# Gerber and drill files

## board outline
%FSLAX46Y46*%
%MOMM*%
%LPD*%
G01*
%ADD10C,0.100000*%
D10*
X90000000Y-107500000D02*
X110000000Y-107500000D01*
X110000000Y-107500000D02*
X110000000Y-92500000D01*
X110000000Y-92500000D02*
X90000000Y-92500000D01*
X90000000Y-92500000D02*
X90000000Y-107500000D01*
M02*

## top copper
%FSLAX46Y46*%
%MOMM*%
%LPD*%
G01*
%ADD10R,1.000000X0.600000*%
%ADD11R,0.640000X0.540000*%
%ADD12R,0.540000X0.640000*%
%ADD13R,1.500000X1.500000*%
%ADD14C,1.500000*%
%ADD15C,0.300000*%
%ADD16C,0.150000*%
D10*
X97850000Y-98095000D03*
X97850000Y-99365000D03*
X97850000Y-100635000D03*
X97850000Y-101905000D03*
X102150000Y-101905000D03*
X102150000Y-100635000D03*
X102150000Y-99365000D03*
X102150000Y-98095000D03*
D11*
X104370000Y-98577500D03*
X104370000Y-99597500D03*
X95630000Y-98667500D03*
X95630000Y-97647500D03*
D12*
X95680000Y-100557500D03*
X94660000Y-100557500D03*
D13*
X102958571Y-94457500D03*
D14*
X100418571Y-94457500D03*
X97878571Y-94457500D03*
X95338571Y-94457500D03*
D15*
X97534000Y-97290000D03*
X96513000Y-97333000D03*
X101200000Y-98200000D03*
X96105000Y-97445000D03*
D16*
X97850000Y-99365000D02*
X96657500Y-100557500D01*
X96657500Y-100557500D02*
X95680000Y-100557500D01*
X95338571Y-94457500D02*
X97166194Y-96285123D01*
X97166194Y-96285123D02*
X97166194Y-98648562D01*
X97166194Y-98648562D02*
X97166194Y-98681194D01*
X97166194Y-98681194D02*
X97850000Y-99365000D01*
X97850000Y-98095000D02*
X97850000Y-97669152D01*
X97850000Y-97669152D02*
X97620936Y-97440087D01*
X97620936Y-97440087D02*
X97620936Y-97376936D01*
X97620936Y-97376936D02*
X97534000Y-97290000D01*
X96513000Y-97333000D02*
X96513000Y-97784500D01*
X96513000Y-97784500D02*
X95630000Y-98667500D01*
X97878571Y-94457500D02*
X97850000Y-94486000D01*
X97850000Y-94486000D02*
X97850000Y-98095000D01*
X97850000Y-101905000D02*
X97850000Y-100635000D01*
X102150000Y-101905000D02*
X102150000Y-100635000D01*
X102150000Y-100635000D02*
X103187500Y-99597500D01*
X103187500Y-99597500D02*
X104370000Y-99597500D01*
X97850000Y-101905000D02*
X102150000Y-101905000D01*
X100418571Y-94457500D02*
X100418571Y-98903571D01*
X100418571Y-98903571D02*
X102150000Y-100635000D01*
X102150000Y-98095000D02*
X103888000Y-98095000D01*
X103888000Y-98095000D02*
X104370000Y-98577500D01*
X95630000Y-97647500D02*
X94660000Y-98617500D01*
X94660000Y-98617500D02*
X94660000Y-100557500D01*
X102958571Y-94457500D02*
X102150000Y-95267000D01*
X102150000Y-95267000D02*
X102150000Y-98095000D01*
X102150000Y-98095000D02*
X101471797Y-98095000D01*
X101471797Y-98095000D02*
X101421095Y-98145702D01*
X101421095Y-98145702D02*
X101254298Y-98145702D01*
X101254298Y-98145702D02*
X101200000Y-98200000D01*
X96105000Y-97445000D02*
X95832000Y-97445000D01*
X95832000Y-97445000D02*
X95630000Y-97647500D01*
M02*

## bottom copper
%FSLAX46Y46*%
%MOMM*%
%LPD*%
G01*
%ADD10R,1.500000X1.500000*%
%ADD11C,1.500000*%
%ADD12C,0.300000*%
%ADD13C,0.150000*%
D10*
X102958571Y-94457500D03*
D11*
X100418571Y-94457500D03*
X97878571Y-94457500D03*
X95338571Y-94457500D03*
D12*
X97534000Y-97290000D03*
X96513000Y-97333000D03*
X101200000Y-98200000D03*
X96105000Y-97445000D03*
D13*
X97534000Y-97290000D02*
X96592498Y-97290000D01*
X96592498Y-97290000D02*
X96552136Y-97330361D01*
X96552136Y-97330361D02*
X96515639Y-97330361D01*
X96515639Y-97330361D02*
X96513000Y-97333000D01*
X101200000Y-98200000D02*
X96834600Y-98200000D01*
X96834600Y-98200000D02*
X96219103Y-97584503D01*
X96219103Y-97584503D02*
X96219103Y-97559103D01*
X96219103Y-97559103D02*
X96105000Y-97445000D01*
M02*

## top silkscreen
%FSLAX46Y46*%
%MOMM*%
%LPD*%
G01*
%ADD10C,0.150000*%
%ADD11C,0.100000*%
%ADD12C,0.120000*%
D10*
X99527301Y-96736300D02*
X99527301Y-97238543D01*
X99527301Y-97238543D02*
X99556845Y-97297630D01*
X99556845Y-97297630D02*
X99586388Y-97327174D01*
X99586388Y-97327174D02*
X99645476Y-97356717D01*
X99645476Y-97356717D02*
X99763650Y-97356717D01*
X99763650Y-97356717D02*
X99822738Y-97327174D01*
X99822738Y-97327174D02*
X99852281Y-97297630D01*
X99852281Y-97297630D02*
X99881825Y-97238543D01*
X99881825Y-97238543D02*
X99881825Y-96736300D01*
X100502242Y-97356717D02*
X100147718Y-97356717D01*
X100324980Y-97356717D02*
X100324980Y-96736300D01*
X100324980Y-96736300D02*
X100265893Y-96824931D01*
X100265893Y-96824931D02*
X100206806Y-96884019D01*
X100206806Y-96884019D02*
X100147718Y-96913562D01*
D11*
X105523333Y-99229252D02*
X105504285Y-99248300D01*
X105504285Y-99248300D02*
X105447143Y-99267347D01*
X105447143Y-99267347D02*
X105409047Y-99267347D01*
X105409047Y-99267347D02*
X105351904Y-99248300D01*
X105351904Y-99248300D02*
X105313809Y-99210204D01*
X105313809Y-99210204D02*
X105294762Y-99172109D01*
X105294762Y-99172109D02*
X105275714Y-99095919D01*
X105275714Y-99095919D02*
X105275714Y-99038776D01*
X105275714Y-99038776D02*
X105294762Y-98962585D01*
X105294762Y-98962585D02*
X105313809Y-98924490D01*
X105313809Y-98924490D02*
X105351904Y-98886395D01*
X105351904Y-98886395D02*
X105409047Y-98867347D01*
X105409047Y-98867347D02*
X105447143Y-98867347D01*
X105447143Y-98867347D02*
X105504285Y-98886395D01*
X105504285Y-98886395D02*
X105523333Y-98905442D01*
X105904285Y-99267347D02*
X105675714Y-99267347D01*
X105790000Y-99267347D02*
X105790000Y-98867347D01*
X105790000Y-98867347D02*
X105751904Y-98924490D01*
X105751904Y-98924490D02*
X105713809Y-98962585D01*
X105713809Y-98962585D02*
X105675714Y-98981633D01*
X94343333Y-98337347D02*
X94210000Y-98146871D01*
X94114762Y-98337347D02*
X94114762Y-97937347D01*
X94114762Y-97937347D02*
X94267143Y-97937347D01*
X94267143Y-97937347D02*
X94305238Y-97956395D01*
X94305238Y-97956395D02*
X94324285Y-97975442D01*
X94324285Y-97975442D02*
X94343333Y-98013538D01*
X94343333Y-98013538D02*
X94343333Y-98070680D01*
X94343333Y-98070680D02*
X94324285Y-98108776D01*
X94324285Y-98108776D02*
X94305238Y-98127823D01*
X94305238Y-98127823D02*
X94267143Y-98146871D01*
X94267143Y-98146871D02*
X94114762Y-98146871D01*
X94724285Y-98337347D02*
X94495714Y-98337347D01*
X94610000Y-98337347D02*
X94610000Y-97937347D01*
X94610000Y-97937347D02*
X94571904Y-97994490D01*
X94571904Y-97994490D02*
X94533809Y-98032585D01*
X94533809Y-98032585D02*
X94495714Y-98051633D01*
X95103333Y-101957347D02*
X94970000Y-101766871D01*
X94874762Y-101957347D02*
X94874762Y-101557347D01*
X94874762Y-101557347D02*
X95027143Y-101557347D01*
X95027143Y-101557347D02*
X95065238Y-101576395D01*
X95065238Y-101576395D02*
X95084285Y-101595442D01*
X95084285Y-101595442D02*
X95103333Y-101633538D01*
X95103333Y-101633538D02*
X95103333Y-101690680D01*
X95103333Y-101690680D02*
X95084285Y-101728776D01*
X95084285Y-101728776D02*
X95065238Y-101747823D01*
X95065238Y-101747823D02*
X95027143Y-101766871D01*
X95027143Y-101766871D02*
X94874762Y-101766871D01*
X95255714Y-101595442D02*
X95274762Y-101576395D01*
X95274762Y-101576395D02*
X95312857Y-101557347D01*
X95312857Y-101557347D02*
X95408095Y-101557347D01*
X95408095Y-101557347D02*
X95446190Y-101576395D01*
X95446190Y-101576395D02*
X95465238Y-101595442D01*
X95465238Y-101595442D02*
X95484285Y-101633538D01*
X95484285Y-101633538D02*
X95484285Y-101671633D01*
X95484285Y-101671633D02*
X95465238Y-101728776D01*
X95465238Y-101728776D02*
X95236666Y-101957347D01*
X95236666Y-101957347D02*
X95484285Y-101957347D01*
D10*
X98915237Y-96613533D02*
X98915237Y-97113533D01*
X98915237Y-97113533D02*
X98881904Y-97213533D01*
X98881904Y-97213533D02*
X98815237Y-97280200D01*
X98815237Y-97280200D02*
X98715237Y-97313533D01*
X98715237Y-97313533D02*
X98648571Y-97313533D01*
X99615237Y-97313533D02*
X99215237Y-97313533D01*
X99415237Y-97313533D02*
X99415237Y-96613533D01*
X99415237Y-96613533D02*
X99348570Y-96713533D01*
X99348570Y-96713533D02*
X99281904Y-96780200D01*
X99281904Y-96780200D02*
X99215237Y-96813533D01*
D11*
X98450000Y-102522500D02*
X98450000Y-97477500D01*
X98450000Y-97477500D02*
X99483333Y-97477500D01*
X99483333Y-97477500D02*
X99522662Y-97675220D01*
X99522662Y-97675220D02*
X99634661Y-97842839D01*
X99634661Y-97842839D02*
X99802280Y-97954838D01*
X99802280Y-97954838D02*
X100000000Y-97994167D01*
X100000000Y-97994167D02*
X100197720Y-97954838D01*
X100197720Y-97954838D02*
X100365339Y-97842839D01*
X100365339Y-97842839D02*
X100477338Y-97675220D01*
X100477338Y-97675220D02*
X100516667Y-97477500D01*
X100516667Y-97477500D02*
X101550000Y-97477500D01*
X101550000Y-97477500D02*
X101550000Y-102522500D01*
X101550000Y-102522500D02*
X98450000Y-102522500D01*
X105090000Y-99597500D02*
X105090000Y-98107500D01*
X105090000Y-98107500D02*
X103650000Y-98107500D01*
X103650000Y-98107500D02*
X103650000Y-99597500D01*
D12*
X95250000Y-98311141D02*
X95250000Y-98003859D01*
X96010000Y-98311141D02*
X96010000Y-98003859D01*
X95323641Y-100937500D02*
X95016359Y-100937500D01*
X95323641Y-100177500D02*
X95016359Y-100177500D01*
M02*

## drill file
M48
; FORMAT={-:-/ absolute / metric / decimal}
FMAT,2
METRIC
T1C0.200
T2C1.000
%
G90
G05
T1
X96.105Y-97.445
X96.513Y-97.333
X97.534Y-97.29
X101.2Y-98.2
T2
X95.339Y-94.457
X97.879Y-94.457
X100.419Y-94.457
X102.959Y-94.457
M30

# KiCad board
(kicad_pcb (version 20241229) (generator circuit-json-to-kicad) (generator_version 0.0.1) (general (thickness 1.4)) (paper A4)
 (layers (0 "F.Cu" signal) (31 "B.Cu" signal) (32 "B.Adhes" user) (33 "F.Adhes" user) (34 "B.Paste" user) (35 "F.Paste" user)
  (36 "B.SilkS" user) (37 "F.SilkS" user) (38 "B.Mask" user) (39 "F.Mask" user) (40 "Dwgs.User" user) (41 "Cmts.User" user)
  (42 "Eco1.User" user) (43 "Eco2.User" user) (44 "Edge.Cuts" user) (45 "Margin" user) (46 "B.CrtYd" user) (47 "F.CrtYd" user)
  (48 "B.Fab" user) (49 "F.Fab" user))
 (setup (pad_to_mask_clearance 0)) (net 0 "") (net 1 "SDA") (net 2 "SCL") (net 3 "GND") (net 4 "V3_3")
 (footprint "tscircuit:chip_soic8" (layer F.Cu) (at 100 100 0)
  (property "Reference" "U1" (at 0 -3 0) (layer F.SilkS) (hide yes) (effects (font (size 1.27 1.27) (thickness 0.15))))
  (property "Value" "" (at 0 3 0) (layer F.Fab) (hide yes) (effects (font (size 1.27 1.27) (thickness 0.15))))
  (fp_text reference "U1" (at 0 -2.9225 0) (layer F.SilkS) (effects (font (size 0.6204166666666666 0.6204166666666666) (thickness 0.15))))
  (fp_line (start -1.5499999999999998 2.5225) (end -1.5499999999999998 -2.5225) (stroke (width 0.1) (type default)) (layer F.SilkS))
  (fp_line (start -1.5499999999999998 -2.5225) (end -0.5166666666666666 -2.5225) (stroke (width 0.1) (type default)) (layer F.SilkS))
  (fp_line (start -0.5166666666666666 -2.5225) (end -0.47733775846416476 -2.32478022661137) (stroke (width 0.1) (type default))
   (layer F.SilkS))
  (fp_line (start -0.47733775846416476 -2.32478022661137) (end -0.3653385036130495 -2.1571614963869505) (stroke (width 0.1) (type default))
   (layer F.SilkS))
  (fp_line (start -0.3653385036130495 -2.1571614963869505) (end -0.19771977338862967 -2.0451622415358353)
   (stroke (width 0.1) (type default)) (layer F.SilkS))
  (fp_line (start -0.19771977338862967 -2.0451622415358353) (end 3.1636708977973285e-17 -2.0058333333333334)
   (stroke (width 0.1) (type default)) (layer F.SilkS))
  (fp_line (start 3.1636708977973285e-17 -2.0058333333333334) (end 0.1977197733886297 -2.0451622415358353)
   (stroke (width 0.1) (type default)) (layer F.SilkS))
  (fp_line (start 0.1977197733886297 -2.0451622415358353) (end 0.3653385036130496 -2.1571614963869505) (stroke (width 0.1) (type default))
   (layer F.SilkS))
  (fp_line (start 0.3653385036130496 -2.1571614963869505) (end 0.47733775846416476 -2.32478022661137) (stroke (width 0.1) (type default))
   (layer F.SilkS))
  (fp_line (start 0.47733775846416476 -2.32478022661137) (end 0.5166666666666666 -2.5225) (stroke (width 0.1) (type default))
   (layer F.SilkS))
  (fp_line (start 0.5166666666666666 -2.5225) (end 1.5499999999999998 -2.5225) (stroke (width 0.1) (type default)) (layer F.SilkS))
  (fp_line (start 1.5499999999999998 -2.5225) (end 1.5499999999999998 2.5225) (stroke (width 0.1) (type default)) (layer F.SilkS))
  (fp_line (start 1.5499999999999998 2.5225) (end -1.5499999999999998 2.5225) (stroke (width 0.1) (type default)) (layer F.SilkS))
  (pad "1" smd rect (at -2.15 -1.905 0) (size 1 0.6) (layers F.Cu F.Paste F.Mask) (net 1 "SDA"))
  (pad "2" smd rect (at -2.15 -0.635 0) (size 1 0.6) (layers F.Cu F.Paste F.Mask) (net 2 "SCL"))
  (pad "3" smd rect (at -2.15 0.635 0) (size 1 0.6) (layers F.Cu F.Paste F.Mask) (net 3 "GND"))
  (pad "4" smd rect (at -2.15 1.905 0) (size 1 0.6) (layers F.Cu F.Paste F.Mask) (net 3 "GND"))
  (pad "5" smd rect (at 2.15 1.905 0) (size 1 0.6) (layers F.Cu F.Paste F.Mask) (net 3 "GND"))
  (pad "6" smd rect (at 2.15 0.635 0) (size 1 0.6) (layers F.Cu F.Paste F.Mask) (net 3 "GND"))
  (pad "7" smd rect (at 2.15 -0.635 0) (size 1 0.6) (layers F.Cu F.Paste F.Mask))
  (pad "8" smd rect (at 2.15 -1.905 0) (size 1 0.6) (layers F.Cu F.Paste F.Mask) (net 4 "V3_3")))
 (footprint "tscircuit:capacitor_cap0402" (layer F.Cu) (at 104.37 99.0875 -90.00000000000001)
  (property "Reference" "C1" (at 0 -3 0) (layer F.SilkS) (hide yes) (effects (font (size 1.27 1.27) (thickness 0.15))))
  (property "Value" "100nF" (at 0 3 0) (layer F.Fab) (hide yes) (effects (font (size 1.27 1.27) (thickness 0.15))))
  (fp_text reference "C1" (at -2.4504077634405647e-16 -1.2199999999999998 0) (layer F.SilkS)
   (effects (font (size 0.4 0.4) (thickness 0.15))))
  (fp_line (start 0.5099999999999999 -0.72) (end -0.9800000000000002 -0.7199999999999994) (stroke (width 0.1) (type default))
   (layer F.SilkS))
  (fp_line (start -0.9800000000000002 -0.7199999999999994) (end -0.9799999999999998 0.7200000000000001) (stroke (width 0.1) (type default))
   (layer F.SilkS))
  (fp_line (start -0.9799999999999998 0.7200000000000001) (end 0.5100000000000001 0.72) (stroke (width 0.1) (type default)) (layer F.SilkS))
  (pad "1" smd rect (at -0.5100000000000001 8.881784197001252e-16 0) (size 0.64 0.54) (layers F.Cu F.Paste F.Mask) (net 4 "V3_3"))
  (pad "2" smd rect (at 0.51 0 0) (size 0.64 0.54) (layers F.Cu F.Paste F.Mask) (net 3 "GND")))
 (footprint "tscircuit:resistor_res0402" (layer F.Cu) (at 95.63 98.1575 90)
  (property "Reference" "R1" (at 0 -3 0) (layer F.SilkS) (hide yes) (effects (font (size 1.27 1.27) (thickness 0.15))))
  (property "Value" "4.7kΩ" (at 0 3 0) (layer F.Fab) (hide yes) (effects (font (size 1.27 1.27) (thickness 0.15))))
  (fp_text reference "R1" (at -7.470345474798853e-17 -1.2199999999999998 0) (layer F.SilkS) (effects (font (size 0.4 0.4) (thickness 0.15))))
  (fp_line (start -0.15364099999999994 -0.3799999999999999) (end 0.1536409999999999 -0.3799999999999999)
   (stroke (width 0.12) (type default)) (layer F.SilkS))
  (fp_line (start -0.1536409999999999 0.3799999999999999) (end 0.15364099999999994 0.3799999999999999) (stroke (width 0.12) (type default))
   (layer F.SilkS))
  (pad "1" smd rect (at -0.51 0 0) (size 0.64 0.54) (layers F.Cu F.Paste F.Mask) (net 1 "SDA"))
  (pad "2" smd rect (at 0.51 0 0) (size 0.64 0.54) (layers F.Cu F.Paste F.Mask) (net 4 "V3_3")))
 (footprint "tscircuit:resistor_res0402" (layer F.Cu) (at 95.17 100.5575 180)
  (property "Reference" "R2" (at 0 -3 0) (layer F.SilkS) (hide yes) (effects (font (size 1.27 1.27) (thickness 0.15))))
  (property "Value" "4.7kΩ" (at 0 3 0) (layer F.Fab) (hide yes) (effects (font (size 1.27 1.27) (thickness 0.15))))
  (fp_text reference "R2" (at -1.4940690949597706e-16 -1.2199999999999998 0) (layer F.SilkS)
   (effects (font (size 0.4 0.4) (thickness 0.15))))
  (fp_line (start -0.15364100000000042 -0.38) (end 0.1536410000000003 -0.38) (stroke (width 0.12) (type default)) (layer F.SilkS))
  (fp_line (start -0.1536410000000003 0.38) (end 0.15364100000000042 0.38) (stroke (width 0.12) (type default)) (layer F.SilkS))
  (pad "1" smd rect (at -0.5099999999999998 -1.1102230246251565e-16 0) (size 0.54 0.64) (layers F.Cu F.Paste F.Mask) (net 2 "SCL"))
  (pad "2" smd rect (at 0.5099999999999998 0 0) (size 0.54 0.64) (layers F.Cu F.Paste F.Mask) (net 4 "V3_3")))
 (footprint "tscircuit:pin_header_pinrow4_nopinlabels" (layer F.Cu) (at 99.14857142857143 94.4575 180)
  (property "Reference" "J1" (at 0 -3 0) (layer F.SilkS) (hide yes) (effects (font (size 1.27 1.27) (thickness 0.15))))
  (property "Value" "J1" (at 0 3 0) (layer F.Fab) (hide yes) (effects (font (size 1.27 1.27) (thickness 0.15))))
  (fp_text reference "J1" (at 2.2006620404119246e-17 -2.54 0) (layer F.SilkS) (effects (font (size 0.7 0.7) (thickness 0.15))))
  (pad "1" thru_hole rect (at -3.81 -4.215879892249837e-16 0) (size 1.5 1.5) (drill 1) (layers *.Cu *.Mask) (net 4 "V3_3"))
  (pad "2" thru_hole circle (at -1.27 1.5553014349171386e-16 0) (size 1.5 1.5) (drill 1) (layers *.Cu *.Mask) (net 3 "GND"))
  (pad "3" thru_hole circle (at 1.27 -1.5553014349171386e-16 0) (size 1.5 1.5) (drill 1) (layers *.Cu *.Mask) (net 1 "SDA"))
  (pad "4" thru_hole circle (at 3.8100000000000005 4.215879892249836e-16 0) (size 1.5 1.5) (drill 1) (layers *.Cu *.Mask) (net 2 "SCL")))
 (segment (start 97.85 99.365) (end 96.6575 100.5575) (width 0.15) (layer F.Cu) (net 2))
 (segment (start 96.6575 100.5575) (end 95.68 100.5575) (width 0.15) (layer F.Cu) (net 2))
 (segment (start 95.33857142857143 94.4575) (end 97.16619411153931 96.28512268296788) (width 0.15) (layer F.Cu) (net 2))
 (segment (start 97.16619411153931 96.28512268296788) (end 97.16619411153931 98.64856177257222) (width 0.15) (layer F.Cu) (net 2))
 (segment (start 97.16619411153931 98.64856177257222) (end 97.16619411153931 98.68119411153931) (width 0.15) (layer F.Cu) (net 2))
 (segment (start 97.16619411153931 98.68119411153931) (end 97.85 99.365) (width 0.15) (layer F.Cu) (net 2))
 (segment (start 97.85 98.095) (end 97.85 97.66915157265616) (width 0.15) (layer F.Cu) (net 1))
 (segment (start 97.85 97.66915157265616) (end 97.62093550613967 97.44008707879584) (width 0.15) (layer F.Cu) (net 1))
 (segment (start 97.62093550613967 97.44008707879584) (end 97.62093550613967 97.37693550613967) (width 0.15) (layer F.Cu) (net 1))
 (segment (start 97.62093550613967 97.37693550613967) (end 97.534 97.29) (width 0.15) (layer F.Cu) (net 1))
 (segment (start 97.534 97.29) (end 96.59249752067976 97.29) (width 0.15) (layer B.Cu) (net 1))
 (segment (start 96.59249752067976 97.29) (end 96.55213608932827 97.33036143135148) (width 0.15) (layer B.Cu) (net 1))
 (segment (start 96.55213608932827 97.33036143135148) (end 96.51563856864853 97.33036143135148) (width 0.15) (layer B.Cu) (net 1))
 (segment (start 96.51563856864853 97.33036143135148) (end 96.513 97.333) (width 0.15) (layer B.Cu) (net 1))
 (segment (start 96.513 97.333) (end 96.513 97.7845) (width 0.15) (layer F.Cu) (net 1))
 (segment (start 96.513 97.7845) (end 95.63 98.6675) (width 0.15) (layer F.Cu) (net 1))
 (segment (start 97.87857142857143 94.4575) (end 97.85 94.486) (width 0.15) (layer F.Cu) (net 1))
 (segment (start 97.85 94.486) (end 97.85 98.095) (width 0.15) (layer F.Cu) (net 1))
 (segment (start 97.85 101.905) (end 97.85 100.635) (width 0.15) (layer F.Cu) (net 3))
 (segment (start 102.15 101.905) (end 102.15 100.635) (width 0.15) (layer F.Cu) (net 3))
 (segment (start 102.15 100.635) (end 103.1875 99.5975) (width 0.15) (layer F.Cu) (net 3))
 (segment (start 103.1875 99.5975) (end 104.37 99.5975) (width 0.15) (layer F.Cu) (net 3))
 (segment (start 97.85 101.905) (end 102.15 101.905) (width 0.15) (layer F.Cu) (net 3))
 (segment (start 100.41857142857143 94.4575) (end 100.41857142857143 98.90357142857142) (width 0.15) (layer F.Cu) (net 3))
 (segment (start 100.41857142857143 98.90357142857142) (end 102.15 100.635) (width 0.15) (layer F.Cu) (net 3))
 (segment (start 102.15 98.095) (end 103.888 98.095) (width 0.15) (layer F.Cu) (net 4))
 (segment (start 103.888 98.095) (end 104.37 98.5775) (width 0.15) (layer F.Cu) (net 4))
 (segment (start 95.63 97.6475) (end 94.66 98.61749999999999) (width 0.15) (layer F.Cu) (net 4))
 (segment (start 94.66 98.61749999999999) (end 94.66 100.5575) (width 0.15) (layer F.Cu) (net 4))
 (segment (start 102.95857142857143 94.4575) (end 102.15 95.267) (width 0.15) (layer F.Cu) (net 4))
 (segment (start 102.15 95.267) (end 102.15 98.095) (width 0.15) (layer F.Cu) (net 4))
 (segment (start 102.15 98.095) (end 101.47179692434212 98.095) (width 0.15) (layer F.Cu) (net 4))
 (segment (start 101.47179692434212 98.095) (end 101.42109493579291 98.1457019885492) (width 0.15) (layer F.Cu) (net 4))
 (segment (start 101.42109493579291 98.1457019885492) (end 101.25429801145079 98.1457019885492) (width 0.15) (layer F.Cu) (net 4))
 (segment (start 101.25429801145079 98.1457019885492) (end 101.2 98.2) (width 0.15) (layer F.Cu) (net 4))
 (segment (start 101.2 98.2) (end 96.83460026614705 98.2) (width 0.15) (layer B.Cu) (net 4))
 (segment (start 96.83460026614705 98.2) (end 96.21910322193693 97.58450295578987) (width 0.15) (layer B.Cu) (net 4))
 (segment (start 96.21910322193693 97.58450295578987) (end 96.21910322193693 97.55910322193692) (width 0.15) (layer B.Cu) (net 4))
 (segment (start 96.21910322193693 97.55910322193692) (end 96.105 97.445) (width 0.15) (layer B.Cu) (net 4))
 (segment (start 96.105 97.445) (end 95.832 97.445) (width 0.15) (layer F.Cu) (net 4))
 (segment (start 95.832 97.445) (end 95.63 97.6475) (width 0.15) (layer F.Cu) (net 4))
 (gr_line (start 90 107.5) (end 110 107.5) (width 0.1) (layer Edge.Cuts))
 (gr_line (start 110 107.5) (end 110 92.5) (width 0.1) (layer Edge.Cuts))
 (gr_line (start 110 92.5) (end 90 92.5) (width 0.1) (layer Edge.Cuts))
 (gr_line (start 90 92.5) (end 90 107.5) (width 0.1) (layer Edge.Cuts))
 (via (at 97.534 97.29) (size 0.3) (drill 0.2) (layers F.Cu B.Cu) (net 1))
 (via (at 96.513 97.333) (size 0.3) (drill 0.2) (layers F.Cu B.Cu) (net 1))
 (via (at 101.2 98.2) (size 0.3) (drill 0.2) (layers F.Cu B.Cu) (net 4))
 (via (at 96.105 97.445) (size 0.3) (drill 0.2) (layers F.Cu B.Cu) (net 4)))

